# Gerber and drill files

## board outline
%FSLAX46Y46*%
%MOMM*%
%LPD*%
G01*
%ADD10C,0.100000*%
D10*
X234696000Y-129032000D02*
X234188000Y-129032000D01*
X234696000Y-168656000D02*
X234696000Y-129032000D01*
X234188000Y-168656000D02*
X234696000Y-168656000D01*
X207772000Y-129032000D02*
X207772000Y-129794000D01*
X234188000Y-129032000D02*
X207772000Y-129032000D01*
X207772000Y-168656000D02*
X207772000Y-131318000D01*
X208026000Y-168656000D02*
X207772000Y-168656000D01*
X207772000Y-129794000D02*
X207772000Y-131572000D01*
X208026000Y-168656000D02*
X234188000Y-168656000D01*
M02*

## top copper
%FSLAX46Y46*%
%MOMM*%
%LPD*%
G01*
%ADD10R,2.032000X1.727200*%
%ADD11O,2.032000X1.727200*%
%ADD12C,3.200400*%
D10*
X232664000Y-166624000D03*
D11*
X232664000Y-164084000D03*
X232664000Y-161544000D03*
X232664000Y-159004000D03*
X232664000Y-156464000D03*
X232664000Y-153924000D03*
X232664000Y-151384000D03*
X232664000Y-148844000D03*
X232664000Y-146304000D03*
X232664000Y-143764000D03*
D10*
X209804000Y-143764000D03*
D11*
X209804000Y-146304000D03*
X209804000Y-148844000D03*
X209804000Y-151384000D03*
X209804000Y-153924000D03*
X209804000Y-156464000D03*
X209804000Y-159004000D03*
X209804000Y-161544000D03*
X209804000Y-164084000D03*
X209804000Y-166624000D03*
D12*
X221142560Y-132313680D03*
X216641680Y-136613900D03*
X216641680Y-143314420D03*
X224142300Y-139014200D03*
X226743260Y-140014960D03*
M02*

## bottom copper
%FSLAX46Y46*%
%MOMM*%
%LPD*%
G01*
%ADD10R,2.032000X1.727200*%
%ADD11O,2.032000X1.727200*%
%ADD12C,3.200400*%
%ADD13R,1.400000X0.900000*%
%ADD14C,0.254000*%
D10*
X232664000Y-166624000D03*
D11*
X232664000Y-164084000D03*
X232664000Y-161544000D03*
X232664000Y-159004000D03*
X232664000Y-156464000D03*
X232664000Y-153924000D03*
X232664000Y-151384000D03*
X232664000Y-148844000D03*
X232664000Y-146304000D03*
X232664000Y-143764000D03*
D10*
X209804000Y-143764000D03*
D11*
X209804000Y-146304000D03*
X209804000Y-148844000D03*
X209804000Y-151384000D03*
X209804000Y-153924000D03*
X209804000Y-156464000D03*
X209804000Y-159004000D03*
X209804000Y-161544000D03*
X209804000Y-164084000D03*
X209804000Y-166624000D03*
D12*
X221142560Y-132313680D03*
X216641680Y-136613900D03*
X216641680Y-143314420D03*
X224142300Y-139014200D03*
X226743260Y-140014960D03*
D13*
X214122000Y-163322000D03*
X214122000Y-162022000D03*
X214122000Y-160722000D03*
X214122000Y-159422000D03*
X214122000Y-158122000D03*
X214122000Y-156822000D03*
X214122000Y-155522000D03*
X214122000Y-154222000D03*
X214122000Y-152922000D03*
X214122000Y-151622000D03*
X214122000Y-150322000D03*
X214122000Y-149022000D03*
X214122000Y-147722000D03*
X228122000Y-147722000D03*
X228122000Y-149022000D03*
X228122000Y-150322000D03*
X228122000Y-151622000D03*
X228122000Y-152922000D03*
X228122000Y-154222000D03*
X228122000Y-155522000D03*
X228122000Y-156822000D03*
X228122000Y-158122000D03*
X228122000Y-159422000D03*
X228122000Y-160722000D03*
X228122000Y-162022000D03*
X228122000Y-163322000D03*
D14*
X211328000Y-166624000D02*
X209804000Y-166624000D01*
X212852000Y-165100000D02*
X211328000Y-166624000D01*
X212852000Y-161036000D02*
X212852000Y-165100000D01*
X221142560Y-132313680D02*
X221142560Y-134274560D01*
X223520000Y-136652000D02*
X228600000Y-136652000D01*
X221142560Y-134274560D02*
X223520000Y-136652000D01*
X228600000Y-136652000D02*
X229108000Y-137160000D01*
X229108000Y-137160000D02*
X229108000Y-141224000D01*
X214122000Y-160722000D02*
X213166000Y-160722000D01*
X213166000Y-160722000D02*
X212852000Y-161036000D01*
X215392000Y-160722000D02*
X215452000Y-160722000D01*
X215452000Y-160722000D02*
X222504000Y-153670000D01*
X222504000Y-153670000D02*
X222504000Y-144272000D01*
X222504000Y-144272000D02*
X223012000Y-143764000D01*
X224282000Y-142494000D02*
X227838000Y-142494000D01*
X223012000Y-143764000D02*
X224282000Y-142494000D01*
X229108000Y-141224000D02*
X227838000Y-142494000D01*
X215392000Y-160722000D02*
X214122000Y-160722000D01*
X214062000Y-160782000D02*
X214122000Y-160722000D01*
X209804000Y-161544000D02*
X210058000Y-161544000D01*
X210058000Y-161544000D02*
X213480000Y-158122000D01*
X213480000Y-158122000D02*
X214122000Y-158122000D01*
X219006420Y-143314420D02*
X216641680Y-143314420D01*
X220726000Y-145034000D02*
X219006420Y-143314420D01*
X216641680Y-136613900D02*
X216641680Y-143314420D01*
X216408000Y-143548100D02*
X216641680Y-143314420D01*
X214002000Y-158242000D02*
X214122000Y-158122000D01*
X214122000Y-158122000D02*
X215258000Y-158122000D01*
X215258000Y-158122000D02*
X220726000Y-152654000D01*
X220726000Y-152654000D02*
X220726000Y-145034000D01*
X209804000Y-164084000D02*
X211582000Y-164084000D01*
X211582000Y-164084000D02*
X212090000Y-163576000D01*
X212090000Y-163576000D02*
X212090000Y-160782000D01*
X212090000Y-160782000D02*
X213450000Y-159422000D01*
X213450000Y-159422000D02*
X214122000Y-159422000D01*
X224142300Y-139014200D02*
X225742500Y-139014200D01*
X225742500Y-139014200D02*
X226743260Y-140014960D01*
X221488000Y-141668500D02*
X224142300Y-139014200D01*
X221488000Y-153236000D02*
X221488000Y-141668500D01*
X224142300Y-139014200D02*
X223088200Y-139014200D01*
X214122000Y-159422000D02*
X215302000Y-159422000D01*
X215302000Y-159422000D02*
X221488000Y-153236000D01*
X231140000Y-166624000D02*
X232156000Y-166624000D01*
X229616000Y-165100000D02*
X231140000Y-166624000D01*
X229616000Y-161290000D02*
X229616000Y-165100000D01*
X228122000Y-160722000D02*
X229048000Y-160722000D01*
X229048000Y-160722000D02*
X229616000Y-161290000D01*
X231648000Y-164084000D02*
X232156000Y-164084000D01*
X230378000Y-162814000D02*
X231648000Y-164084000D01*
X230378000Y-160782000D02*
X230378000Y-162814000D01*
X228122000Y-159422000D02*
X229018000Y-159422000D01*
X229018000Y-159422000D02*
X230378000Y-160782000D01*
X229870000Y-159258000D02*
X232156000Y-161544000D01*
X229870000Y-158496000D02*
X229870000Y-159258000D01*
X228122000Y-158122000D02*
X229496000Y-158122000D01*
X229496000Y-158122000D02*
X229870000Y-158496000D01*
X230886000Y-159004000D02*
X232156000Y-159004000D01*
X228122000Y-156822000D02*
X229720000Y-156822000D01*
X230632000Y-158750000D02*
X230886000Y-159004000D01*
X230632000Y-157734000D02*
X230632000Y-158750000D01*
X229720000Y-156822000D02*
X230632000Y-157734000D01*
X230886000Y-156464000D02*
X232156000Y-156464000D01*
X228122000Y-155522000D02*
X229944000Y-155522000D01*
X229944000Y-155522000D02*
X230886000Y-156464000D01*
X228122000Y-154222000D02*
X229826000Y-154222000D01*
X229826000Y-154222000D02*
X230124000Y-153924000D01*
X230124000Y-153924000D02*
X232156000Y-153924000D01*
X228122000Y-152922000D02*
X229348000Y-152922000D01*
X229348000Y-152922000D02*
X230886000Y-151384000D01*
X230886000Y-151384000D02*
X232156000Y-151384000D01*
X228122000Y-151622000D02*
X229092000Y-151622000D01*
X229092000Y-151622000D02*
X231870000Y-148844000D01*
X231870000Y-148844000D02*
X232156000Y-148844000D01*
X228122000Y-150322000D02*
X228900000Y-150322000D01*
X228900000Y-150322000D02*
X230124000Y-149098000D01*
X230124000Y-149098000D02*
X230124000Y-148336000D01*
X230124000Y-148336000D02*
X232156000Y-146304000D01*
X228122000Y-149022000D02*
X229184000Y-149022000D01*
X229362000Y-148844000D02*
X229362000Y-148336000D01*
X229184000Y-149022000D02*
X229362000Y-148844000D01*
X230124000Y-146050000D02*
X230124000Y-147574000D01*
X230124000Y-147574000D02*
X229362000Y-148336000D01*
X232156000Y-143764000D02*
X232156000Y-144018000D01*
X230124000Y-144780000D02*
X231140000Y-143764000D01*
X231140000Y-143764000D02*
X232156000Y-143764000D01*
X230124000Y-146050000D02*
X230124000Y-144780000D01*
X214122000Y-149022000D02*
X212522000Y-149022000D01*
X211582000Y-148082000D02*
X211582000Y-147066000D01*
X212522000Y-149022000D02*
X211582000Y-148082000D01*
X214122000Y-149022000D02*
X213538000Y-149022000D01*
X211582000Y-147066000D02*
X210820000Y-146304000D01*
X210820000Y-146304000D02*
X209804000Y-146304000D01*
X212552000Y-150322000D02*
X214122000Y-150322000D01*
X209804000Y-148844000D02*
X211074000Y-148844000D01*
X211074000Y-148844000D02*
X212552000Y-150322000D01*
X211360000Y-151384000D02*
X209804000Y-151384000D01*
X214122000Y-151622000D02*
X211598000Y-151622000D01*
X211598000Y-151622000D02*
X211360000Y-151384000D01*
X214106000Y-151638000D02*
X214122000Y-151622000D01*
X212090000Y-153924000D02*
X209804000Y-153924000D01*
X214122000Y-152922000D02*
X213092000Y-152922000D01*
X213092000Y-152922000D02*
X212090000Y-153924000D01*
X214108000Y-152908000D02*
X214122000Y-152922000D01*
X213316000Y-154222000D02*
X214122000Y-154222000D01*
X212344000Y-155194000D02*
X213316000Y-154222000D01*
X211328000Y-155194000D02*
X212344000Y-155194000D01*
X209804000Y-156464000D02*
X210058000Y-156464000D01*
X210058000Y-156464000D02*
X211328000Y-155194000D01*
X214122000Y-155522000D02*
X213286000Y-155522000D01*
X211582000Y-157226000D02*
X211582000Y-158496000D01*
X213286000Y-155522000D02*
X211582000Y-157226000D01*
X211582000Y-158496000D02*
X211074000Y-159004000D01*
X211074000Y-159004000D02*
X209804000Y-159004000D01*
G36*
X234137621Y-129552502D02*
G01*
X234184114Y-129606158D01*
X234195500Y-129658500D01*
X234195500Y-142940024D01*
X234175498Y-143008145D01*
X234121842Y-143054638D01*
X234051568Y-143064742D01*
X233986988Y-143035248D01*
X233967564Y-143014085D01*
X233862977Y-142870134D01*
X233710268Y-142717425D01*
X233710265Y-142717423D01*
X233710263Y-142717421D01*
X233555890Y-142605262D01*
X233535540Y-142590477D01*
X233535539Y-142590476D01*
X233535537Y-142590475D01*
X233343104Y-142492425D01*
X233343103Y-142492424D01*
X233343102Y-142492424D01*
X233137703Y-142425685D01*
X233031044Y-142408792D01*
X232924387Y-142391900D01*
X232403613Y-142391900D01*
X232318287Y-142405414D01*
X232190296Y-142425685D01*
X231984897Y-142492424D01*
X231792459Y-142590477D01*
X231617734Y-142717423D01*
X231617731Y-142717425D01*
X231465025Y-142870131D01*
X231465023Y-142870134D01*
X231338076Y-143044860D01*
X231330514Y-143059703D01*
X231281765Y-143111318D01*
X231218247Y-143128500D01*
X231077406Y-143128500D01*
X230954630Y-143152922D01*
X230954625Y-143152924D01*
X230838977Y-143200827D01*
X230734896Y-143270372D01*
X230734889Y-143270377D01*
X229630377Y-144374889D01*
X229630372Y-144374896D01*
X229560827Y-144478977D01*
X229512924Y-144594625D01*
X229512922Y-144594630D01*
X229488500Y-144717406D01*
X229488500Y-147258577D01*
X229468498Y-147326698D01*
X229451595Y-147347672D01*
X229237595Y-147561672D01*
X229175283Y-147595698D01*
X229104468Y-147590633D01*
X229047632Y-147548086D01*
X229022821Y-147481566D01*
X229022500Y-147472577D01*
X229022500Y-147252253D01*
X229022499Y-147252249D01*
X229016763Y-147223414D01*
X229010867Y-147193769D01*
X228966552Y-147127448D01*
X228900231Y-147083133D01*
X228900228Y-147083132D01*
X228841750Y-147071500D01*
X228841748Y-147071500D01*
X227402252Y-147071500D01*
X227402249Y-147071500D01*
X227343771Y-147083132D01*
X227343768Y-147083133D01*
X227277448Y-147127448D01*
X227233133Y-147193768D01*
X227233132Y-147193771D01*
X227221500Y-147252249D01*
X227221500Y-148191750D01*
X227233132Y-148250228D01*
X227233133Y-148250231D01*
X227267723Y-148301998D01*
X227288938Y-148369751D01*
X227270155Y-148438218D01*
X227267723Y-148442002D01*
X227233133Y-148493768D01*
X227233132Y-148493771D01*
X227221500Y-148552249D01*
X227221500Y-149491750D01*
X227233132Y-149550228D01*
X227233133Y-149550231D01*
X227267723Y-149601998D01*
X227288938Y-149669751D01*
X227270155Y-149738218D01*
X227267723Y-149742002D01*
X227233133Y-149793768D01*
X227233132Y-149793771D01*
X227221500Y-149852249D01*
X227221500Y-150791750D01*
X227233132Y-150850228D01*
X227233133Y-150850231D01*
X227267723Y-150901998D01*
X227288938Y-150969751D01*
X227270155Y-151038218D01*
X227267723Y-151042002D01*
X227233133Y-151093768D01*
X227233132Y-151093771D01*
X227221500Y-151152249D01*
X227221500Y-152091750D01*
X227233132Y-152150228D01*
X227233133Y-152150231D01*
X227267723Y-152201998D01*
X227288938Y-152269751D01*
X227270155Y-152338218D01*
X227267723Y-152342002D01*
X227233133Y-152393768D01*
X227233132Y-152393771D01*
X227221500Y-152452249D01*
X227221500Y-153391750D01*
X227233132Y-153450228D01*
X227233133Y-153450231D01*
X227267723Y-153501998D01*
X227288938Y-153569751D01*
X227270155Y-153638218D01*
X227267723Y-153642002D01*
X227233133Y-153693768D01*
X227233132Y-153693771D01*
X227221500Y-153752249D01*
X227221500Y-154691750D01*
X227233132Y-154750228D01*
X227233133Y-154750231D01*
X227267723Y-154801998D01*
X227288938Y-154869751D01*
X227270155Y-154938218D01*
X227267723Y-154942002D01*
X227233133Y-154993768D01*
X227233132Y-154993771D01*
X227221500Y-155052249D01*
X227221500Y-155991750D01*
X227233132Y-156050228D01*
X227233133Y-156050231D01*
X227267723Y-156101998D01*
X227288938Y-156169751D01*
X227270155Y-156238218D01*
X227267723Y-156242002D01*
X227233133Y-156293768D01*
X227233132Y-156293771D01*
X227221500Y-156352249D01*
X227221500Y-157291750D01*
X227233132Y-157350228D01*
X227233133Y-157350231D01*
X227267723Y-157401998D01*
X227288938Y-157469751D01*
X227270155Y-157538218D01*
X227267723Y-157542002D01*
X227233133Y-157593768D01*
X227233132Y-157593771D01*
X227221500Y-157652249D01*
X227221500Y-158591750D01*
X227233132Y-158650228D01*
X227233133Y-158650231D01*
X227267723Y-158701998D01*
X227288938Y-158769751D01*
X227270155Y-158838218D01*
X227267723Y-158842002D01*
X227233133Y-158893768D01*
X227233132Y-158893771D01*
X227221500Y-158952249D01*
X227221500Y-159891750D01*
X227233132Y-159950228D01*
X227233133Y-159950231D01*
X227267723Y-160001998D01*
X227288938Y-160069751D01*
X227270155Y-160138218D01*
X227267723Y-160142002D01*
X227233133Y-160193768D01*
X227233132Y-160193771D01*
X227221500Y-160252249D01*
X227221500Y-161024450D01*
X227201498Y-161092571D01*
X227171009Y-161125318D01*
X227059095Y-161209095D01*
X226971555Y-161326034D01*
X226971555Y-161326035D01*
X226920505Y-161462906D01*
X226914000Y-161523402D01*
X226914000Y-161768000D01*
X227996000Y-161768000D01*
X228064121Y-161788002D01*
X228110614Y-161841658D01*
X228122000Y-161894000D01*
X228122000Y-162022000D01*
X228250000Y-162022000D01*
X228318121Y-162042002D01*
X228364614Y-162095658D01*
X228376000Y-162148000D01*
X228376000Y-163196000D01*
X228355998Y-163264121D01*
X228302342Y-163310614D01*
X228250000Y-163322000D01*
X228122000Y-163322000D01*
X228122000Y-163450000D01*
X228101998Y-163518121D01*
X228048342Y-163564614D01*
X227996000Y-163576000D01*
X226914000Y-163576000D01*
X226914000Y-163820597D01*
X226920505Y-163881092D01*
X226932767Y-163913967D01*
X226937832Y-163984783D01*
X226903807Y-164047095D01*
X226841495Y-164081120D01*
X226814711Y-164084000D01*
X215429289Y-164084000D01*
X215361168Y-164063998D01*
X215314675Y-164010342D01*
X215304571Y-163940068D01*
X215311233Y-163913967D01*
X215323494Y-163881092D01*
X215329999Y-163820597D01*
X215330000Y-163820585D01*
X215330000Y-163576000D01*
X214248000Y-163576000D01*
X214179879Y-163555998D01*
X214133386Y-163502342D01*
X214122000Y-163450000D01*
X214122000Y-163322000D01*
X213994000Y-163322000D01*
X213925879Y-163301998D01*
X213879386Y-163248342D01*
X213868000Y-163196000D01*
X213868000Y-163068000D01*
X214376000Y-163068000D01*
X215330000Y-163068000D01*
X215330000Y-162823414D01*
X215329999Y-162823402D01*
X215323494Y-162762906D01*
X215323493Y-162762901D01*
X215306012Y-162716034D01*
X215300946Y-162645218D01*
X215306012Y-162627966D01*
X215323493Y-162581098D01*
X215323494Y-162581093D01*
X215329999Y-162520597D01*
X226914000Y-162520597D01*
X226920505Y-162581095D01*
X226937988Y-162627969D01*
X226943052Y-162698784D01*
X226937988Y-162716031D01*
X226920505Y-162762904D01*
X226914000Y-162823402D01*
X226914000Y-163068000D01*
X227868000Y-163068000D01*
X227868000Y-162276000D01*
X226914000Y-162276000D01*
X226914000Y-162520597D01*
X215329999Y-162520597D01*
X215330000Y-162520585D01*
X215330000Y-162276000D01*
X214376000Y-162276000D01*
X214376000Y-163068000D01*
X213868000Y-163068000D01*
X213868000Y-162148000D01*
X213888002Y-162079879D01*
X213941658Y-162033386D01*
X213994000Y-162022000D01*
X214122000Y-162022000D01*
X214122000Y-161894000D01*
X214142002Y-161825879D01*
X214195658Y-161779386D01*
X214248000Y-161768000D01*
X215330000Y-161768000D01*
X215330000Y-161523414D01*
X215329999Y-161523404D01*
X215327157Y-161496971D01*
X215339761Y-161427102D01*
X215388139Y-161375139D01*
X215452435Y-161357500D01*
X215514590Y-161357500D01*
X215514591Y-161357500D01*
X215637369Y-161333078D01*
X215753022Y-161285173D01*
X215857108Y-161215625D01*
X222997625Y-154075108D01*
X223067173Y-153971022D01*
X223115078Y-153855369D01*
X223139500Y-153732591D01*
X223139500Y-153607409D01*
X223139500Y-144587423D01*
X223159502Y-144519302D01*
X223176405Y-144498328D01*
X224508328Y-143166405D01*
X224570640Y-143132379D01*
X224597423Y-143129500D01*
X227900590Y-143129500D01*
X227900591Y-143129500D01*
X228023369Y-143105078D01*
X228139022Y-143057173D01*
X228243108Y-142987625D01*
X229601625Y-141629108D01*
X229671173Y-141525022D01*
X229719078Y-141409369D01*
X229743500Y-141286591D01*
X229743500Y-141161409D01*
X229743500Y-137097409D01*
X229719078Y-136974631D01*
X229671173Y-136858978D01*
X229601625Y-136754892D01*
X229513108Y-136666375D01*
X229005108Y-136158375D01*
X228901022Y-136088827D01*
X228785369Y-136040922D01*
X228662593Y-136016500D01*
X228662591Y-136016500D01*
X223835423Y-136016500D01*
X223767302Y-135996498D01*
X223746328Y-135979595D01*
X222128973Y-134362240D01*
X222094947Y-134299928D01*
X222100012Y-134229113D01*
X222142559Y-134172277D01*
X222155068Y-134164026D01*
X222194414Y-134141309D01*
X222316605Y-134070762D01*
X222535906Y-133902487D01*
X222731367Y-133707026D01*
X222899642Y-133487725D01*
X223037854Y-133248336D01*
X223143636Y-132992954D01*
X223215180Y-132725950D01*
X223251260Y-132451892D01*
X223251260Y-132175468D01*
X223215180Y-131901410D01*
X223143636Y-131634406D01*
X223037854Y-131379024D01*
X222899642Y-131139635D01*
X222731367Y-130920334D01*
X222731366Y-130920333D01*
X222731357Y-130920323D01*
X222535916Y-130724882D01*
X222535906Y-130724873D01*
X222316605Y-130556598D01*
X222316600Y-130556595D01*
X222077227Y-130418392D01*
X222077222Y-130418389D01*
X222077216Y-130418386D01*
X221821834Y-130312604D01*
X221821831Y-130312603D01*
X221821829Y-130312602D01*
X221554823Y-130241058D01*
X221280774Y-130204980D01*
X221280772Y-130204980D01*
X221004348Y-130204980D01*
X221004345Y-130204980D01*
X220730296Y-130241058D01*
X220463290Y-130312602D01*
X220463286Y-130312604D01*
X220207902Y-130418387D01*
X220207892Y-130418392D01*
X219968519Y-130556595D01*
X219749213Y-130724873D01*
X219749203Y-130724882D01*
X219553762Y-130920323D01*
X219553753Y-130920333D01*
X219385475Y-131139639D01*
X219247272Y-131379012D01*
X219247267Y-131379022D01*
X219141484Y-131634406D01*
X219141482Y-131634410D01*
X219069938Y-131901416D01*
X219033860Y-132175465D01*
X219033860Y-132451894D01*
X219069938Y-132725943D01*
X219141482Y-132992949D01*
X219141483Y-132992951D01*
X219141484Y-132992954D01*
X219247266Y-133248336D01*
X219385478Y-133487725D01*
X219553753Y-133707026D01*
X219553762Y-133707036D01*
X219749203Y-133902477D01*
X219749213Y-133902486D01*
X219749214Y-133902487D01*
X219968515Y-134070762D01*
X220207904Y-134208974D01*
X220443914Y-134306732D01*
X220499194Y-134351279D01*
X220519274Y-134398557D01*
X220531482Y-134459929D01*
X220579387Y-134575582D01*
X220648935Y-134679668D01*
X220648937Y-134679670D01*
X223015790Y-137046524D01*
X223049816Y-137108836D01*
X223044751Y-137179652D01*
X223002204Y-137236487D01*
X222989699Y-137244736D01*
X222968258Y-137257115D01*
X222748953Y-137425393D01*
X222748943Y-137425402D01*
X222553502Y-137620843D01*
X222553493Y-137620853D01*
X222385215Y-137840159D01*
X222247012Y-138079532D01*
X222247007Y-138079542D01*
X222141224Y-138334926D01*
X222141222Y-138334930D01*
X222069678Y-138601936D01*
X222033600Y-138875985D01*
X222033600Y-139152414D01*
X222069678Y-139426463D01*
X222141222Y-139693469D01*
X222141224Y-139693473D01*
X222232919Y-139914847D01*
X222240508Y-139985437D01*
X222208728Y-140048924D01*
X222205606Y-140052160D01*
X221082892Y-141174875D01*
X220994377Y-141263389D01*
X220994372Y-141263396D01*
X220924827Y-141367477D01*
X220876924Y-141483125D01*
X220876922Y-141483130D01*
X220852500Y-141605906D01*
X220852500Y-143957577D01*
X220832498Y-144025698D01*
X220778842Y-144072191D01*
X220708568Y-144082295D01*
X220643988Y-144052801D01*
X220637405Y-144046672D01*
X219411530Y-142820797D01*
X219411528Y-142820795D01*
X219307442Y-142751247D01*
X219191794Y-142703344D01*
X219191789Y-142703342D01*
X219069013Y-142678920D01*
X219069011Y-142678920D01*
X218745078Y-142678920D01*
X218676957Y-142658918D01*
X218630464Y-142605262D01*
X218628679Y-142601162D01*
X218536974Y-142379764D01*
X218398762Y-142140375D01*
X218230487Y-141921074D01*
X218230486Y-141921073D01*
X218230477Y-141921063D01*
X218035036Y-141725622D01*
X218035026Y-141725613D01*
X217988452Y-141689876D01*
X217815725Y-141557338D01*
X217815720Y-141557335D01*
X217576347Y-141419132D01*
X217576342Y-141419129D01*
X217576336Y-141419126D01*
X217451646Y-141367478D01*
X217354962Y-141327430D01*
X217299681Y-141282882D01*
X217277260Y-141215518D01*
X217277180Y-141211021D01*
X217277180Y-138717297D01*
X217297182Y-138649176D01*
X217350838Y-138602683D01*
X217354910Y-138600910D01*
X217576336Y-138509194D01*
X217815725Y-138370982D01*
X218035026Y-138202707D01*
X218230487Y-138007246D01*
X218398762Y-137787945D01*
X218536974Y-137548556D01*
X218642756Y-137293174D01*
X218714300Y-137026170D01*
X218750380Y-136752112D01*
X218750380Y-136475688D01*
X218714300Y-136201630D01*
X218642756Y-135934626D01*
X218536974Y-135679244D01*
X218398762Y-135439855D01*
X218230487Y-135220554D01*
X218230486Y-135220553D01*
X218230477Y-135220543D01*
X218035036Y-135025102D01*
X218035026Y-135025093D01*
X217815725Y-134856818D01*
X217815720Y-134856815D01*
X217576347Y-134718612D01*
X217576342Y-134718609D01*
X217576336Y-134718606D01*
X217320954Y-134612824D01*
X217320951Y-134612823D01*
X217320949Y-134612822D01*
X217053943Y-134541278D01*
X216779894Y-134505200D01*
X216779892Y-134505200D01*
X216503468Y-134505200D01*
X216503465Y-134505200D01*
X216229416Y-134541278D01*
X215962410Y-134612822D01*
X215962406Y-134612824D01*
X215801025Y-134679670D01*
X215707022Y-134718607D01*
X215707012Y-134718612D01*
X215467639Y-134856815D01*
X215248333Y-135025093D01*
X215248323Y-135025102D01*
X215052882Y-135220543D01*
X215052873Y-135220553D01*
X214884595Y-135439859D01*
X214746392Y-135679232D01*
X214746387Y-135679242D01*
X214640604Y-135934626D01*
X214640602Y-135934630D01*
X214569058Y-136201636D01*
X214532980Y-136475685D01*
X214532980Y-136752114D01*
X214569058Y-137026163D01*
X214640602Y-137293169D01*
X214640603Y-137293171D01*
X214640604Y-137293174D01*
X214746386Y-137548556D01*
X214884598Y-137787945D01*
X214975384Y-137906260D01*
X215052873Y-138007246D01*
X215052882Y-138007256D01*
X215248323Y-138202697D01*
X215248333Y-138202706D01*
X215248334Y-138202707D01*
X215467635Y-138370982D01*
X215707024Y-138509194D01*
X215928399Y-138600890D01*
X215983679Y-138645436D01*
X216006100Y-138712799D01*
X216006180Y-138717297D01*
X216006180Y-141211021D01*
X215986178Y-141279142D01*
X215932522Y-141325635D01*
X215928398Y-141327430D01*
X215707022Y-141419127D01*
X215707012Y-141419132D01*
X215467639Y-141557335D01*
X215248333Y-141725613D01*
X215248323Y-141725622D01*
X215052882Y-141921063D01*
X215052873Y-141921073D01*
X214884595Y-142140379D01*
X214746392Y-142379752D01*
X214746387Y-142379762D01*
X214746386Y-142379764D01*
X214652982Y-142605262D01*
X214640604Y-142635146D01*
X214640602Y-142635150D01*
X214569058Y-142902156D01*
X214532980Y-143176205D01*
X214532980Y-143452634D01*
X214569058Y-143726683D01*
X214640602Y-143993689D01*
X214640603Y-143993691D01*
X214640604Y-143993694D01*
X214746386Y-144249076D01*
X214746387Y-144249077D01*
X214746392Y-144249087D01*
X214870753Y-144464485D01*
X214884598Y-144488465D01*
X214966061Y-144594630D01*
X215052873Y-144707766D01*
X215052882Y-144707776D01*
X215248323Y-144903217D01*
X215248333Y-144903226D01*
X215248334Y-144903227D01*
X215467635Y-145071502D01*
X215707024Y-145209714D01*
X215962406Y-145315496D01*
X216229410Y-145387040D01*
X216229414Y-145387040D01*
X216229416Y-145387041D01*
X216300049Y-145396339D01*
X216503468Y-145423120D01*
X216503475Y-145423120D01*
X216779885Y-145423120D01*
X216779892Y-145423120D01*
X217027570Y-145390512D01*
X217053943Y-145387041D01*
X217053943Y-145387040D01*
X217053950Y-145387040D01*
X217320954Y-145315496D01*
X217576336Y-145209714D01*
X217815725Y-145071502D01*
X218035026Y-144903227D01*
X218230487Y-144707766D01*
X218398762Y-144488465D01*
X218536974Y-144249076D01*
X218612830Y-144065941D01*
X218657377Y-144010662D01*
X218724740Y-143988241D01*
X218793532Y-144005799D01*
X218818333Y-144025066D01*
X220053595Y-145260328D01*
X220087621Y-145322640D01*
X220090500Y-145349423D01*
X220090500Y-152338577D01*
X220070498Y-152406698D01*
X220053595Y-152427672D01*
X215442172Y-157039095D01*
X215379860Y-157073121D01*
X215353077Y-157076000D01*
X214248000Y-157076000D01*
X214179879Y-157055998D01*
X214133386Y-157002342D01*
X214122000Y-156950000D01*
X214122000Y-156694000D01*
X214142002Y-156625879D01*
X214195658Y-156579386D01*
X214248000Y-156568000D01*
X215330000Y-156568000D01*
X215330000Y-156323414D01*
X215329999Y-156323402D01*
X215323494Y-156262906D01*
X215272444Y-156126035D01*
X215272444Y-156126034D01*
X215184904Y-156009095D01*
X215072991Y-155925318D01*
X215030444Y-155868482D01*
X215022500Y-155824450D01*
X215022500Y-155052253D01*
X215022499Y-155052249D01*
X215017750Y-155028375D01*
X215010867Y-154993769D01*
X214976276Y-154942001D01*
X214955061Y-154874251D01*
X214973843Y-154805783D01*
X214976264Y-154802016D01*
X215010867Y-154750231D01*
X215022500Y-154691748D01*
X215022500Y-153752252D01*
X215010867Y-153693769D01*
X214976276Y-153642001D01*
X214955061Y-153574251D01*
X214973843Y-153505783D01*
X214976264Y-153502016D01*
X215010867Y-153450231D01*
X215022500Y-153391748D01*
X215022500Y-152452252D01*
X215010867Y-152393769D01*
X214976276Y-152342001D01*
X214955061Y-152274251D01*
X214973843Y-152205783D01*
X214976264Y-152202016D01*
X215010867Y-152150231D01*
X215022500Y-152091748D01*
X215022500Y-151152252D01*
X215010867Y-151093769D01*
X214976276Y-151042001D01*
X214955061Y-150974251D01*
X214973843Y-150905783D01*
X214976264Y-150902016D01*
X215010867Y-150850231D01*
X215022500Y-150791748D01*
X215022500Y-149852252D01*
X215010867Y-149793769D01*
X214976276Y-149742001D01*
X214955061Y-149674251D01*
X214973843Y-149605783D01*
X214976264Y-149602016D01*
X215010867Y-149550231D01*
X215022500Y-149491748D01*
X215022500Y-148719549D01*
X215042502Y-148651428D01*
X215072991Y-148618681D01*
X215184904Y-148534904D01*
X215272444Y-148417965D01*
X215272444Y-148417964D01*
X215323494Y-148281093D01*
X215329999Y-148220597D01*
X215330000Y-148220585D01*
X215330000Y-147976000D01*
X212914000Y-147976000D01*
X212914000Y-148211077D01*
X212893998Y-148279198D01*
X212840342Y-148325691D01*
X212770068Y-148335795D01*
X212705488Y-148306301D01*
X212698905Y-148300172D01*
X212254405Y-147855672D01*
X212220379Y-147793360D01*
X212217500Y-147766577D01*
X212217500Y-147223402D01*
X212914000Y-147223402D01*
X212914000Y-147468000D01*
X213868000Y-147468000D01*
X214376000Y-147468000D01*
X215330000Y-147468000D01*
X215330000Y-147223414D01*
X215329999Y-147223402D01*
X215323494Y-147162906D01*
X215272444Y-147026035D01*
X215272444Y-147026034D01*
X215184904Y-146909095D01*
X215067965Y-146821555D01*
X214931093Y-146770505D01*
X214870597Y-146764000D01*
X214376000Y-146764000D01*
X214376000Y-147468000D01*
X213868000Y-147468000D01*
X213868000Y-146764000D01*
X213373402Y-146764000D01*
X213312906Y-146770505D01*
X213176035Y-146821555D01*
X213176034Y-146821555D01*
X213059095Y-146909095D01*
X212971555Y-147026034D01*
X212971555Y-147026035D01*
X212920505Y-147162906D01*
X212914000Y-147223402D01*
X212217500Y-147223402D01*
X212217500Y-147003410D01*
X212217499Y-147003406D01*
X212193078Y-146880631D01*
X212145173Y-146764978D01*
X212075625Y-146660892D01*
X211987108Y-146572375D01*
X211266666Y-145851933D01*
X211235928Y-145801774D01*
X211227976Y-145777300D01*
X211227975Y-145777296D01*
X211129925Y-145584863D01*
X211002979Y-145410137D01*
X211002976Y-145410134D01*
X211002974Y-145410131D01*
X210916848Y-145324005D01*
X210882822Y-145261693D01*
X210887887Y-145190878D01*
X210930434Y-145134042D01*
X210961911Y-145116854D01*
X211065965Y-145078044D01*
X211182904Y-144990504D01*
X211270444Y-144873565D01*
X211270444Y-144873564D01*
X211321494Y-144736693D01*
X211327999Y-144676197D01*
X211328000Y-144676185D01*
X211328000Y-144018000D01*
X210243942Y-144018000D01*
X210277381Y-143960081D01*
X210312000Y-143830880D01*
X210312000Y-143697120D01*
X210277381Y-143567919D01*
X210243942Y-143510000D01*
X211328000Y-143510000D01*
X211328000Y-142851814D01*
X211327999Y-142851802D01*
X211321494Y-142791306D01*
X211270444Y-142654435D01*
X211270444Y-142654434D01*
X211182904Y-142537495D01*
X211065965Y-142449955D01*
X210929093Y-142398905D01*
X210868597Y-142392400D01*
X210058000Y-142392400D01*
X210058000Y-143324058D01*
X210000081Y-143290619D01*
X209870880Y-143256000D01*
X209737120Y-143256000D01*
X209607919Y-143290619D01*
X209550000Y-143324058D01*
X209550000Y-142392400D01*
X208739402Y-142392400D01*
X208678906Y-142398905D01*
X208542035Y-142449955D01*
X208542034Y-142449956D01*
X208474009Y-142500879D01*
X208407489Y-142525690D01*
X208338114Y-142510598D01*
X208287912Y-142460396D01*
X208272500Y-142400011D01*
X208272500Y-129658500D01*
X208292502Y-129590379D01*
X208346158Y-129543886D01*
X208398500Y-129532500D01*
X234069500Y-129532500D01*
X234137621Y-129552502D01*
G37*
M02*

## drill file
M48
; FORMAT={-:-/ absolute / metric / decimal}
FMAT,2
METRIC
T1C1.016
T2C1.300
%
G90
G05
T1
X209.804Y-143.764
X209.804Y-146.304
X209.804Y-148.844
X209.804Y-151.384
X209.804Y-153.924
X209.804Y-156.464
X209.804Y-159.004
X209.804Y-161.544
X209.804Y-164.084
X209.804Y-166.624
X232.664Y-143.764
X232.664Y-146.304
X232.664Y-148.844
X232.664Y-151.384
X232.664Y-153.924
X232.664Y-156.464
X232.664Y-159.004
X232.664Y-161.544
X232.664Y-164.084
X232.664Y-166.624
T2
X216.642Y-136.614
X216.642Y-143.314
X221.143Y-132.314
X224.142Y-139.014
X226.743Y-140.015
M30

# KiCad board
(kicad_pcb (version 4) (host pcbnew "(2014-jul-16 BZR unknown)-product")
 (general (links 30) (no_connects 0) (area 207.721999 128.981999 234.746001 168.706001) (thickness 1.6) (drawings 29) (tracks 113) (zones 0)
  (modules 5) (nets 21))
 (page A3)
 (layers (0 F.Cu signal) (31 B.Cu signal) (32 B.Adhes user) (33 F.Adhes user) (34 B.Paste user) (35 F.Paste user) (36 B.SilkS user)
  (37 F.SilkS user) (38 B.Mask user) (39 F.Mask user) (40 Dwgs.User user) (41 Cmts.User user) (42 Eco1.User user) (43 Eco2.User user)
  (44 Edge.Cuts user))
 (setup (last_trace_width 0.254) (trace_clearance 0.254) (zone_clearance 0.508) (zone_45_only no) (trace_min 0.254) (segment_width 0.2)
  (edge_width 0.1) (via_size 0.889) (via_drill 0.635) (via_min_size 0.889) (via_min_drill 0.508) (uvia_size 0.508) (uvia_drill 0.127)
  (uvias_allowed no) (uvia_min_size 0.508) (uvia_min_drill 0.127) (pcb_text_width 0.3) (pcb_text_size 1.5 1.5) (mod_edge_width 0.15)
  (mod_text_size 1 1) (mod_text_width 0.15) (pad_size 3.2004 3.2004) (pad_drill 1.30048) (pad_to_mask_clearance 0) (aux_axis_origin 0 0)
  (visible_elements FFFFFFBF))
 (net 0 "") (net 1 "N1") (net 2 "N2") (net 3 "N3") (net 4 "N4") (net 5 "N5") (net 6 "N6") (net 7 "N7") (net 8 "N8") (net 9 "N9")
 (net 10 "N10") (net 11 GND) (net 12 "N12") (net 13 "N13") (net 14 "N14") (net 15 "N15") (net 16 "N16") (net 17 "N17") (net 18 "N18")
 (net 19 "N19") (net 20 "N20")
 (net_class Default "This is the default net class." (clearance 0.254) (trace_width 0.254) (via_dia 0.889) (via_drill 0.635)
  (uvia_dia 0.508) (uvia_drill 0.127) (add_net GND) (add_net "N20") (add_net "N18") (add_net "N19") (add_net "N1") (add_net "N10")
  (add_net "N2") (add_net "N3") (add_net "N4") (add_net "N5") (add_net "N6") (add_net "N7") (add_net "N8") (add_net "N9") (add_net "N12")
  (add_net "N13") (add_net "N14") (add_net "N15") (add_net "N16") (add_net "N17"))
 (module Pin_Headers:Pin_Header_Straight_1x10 (layer B.Cu) (at 232.664 155.194 90)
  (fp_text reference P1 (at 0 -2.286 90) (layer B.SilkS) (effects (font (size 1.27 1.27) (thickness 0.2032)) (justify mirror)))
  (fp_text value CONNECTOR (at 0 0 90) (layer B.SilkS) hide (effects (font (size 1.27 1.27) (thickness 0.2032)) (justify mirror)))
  (pad 1 thru_hole rect (at -11.43 0 90) (size 1.7272 2.032) (drill 1.016) (layers *.Cu *.Mask B.SilkS) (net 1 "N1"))
  (pad 2 thru_hole oval (at -8.89 0 90) (size 1.7272 2.032) (drill 1.016) (layers *.Cu *.Mask B.SilkS) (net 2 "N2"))
  (pad 3 thru_hole oval (at -6.35 0 90) (size 1.7272 2.032) (drill 1.016) (layers *.Cu *.Mask B.SilkS) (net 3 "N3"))
  (pad 4 thru_hole oval (at -3.81 0 90) (size 1.7272 2.032) (drill 1.016) (layers *.Cu *.Mask B.SilkS) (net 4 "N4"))
  (pad 5 thru_hole oval (at -1.27 0 90) (size 1.7272 2.032) (drill 1.016) (layers *.Cu *.Mask B.SilkS) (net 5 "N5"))
  (pad 6 thru_hole oval (at 1.27 0 90) (size 1.7272 2.032) (drill 1.016) (layers *.Cu *.Mask B.SilkS) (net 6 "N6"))
  (pad 7 thru_hole oval (at 3.81 0 90) (size 1.7272 2.032) (drill 1.016) (layers *.Cu *.Mask B.SilkS) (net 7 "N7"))
  (pad 8 thru_hole oval (at 6.35 0 90) (size 1.7272 2.032) (drill 1.016) (layers *.Cu *.Mask B.SilkS) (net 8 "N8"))
  (pad 9 thru_hole oval (at 8.89 0 90) (size 1.7272 2.032) (drill 1.016) (layers *.Cu *.Mask B.SilkS) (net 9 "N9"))
  (pad 10 thru_hole oval (at 11.43 0 90) (size 1.7272 2.032) (drill 1.016) (layers *.Cu *.Mask B.SilkS) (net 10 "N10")))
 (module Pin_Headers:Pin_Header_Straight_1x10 (layer B.Cu) (at 209.804 155.194 270)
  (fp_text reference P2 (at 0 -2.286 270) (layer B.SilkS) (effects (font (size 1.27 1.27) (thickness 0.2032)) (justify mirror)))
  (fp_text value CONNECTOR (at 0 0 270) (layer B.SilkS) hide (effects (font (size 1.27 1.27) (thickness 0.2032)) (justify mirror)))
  (pad 1 thru_hole rect (at -11.43 0 270) (size 1.7272 2.032) (drill 1.016) (layers *.Cu *.Mask B.SilkS) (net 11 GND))
  (pad 2 thru_hole oval (at -8.89 0 270) (size 1.7272 2.032) (drill 1.016) (layers *.Cu *.Mask B.SilkS) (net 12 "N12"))
  (pad 3 thru_hole oval (at -6.35 0 270) (size 1.7272 2.032) (drill 1.016) (layers *.Cu *.Mask B.SilkS) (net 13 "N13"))
  (pad 4 thru_hole oval (at -3.81 0 270) (size 1.7272 2.032) (drill 1.016) (layers *.Cu *.Mask B.SilkS) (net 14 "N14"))
  (pad 5 thru_hole oval (at -1.27 0 270) (size 1.7272 2.032) (drill 1.016) (layers *.Cu *.Mask B.SilkS) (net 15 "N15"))
  (pad 6 thru_hole oval (at 1.27 0 270) (size 1.7272 2.032) (drill 1.016) (layers *.Cu *.Mask B.SilkS) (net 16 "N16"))
  (pad 7 thru_hole oval (at 3.81 0 270) (size 1.7272 2.032) (drill 1.016) (layers *.Cu *.Mask B.SilkS) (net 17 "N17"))
  (pad 8 thru_hole oval (at 6.35 0 270) (size 1.7272 2.032) (drill 1.016) (layers *.Cu *.Mask B.SilkS) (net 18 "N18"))
  (pad 9 thru_hole oval (at 8.89 0 270) (size 1.7272 2.032) (drill 1.016) (layers *.Cu *.Mask B.SilkS) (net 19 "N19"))
  (pad 10 thru_hole oval (at 11.43 0 270) (size 1.7272 2.032) (drill 1.016) (layers *.Cu *.Mask B.SilkS) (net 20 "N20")))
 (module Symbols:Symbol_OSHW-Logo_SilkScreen (layer F.Cu) (at 211.582 132.842)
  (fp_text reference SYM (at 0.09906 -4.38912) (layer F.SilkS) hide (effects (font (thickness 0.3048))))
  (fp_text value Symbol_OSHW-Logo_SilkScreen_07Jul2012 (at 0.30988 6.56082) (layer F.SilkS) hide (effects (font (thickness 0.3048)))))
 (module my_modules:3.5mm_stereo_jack (layer F.Cu) (at 221.742 137.414)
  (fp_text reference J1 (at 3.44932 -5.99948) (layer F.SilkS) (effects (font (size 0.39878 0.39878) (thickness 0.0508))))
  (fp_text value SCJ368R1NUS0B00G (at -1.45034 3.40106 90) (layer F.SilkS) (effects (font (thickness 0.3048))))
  (pad 1 thru_hole circle (at -0.59944 -5.10032) (size 3.2004 3.2004) (drill 1.30048) (layers *.Cu *.Mask F.SilkS) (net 20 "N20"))
  (pad 2 thru_hole circle (at -5.10032 -0.8001) (size 3.2004 3.2004) (drill 1.30048) (layers *.Cu *.Mask F.SilkS) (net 18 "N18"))
  (pad 3 thru_hole circle (at -5.10032 5.90042) (size 3.2004 3.2004) (drill 1.30048) (layers *.Cu *.Mask F.SilkS) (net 18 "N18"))
  (pad 5 thru_hole circle (at 2.4003 1.6002) (size 3.2004 3.2004) (drill 1.30048) (layers *.Cu *.Mask F.SilkS) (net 19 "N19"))
  (pad 4 thru_hole circle (at 5.00126 2.60096) (size 3.2004 3.2004) (drill 1.30048) (layers *.Cu *.Mask F.SilkS) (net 19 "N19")))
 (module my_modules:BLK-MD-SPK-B (layer B.Cu) (at 212.852 169.672) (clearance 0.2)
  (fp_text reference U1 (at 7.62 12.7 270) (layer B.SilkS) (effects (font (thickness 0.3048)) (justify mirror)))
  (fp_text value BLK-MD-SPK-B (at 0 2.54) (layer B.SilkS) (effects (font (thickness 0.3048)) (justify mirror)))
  (pad 1 smd rect (at 1.27 -6.35 180) (size 1.4 0.9) (layers B.Cu B.Paste B.Mask) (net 11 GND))
  (pad 2 smd rect (at 1.27 -7.65 180) (size 1.4 0.9) (layers B.Cu B.Paste B.Mask) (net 11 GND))
  (pad 3 smd rect (at 1.27 -8.95 180) (size 1.4 0.9) (layers B.Cu B.Paste B.Mask) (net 20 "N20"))
  (pad 4 smd rect (at 1.27 -10.25 180) (size 1.4 0.9) (layers B.Cu B.Paste B.Mask) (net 19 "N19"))
  (pad 5 smd rect (at 1.27 -11.55 180) (size 1.4 0.9) (layers B.Cu B.Paste B.Mask) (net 18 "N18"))
  (pad 6 smd rect (at 1.27 -12.85 180) (size 1.4 0.9) (layers B.Cu B.Paste B.Mask) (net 11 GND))
  (pad 7 smd rect (at 1.27 -14.15 180) (size 1.4 0.9) (layers B.Cu B.Paste B.Mask) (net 17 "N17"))
  (pad 8 smd rect (at 1.27 -15.45 180) (size 1.4 0.9) (layers B.Cu B.Paste B.Mask) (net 16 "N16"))
  (pad 9 smd rect (at 1.27 -16.75 180) (size 1.4 0.9) (layers B.Cu B.Paste B.Mask) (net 15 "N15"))
  (pad 10 smd rect (at 1.27 -18.05 180) (size 1.4 0.9) (layers B.Cu B.Paste B.Mask) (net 14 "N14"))
  (pad 11 smd rect (at 1.27 -19.35 180) (size 1.4 0.9) (layers B.Cu B.Paste B.Mask) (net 13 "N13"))
  (pad 12 smd rect (at 1.27 -20.65 180) (size 1.4 0.9) (layers B.Cu B.Paste B.Mask) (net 12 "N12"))
  (pad 13 smd rect (at 1.27 -21.95 180) (size 1.4 0.9) (layers B.Cu B.Paste B.Mask) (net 11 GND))
  (pad 14 smd rect (at 15.27 -21.95 180) (size 1.4 0.9) (layers B.Cu B.Paste B.Mask))
  (pad 15 smd rect (at 15.27 -20.65 180) (size 1.4 0.9) (layers B.Cu B.Paste B.Mask) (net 10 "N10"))
  (pad 16 smd rect (at 15.27 -19.35 180) (size 1.4 0.9) (layers B.Cu B.Paste B.Mask) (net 9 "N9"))
  (pad 17 smd rect (at 15.27 -18.05 180) (size 1.4 0.9) (layers B.Cu B.Paste B.Mask) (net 8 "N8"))
  (pad 18 smd rect (at 15.27 -16.75 180) (size 1.4 0.9) (layers B.Cu B.Paste B.Mask) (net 7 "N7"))
  (pad 19 smd rect (at 15.27 -15.45 180) (size 1.4 0.9) (layers B.Cu B.Paste B.Mask) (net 6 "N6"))
  (pad 20 smd rect (at 15.27 -14.15 180) (size 1.4 0.9) (layers B.Cu B.Paste B.Mask) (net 5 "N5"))
  (pad 21 smd rect (at 15.27 -12.85 180) (size 1.4 0.9) (layers B.Cu B.Paste B.Mask) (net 4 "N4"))
  (pad 22 smd rect (at 15.27 -11.55 180) (size 1.4 0.9) (layers B.Cu B.Paste B.Mask) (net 3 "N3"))
  (pad 23 smd rect (at 15.27 -10.25 180) (size 1.4 0.9) (layers B.Cu B.Paste B.Mask) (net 2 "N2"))
  (pad 24 smd rect (at 15.27 -8.95 180) (size 1.4 0.9) (layers B.Cu B.Paste B.Mask) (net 1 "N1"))
  (pad 25 smd rect (at 15.27 -7.65 180) (size 1.4 0.9) (layers B.Cu B.Paste B.Mask) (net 11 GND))
  (pad 26 smd rect (at 15.27 -6.35 180) (size 1.4 0.9) (layers B.Cu B.Paste B.Mask) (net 11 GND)))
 (gr_line (start 234.696 129.032) (end 234.188 129.032) (angle 90) (layer Edge.Cuts) (width 0.1))
 (gr_line (start 234.696 168.656) (end 234.696 129.032) (angle 90) (layer Edge.Cuts) (width 0.1))
 (gr_line (start 234.188 168.656) (end 234.696 168.656) (angle 90) (layer Edge.Cuts) (width 0.1))
 (gr_line (start 207.772 129.032) (end 207.772 129.794) (angle 90) (layer Edge.Cuts) (width 0.1))
 (gr_line (start 234.188 129.032) (end 207.772 129.032) (angle 90) (layer Edge.Cuts) (width 0.1))
 (gr_line (start 207.772 168.656) (end 207.772 131.318) (angle 90) (layer Edge.Cuts) (width 0.1))
 (gr_line (start 208.026 168.656) (end 207.772 168.656) (angle 90) (layer Edge.Cuts) (width 0.1))
 (gr_line (start 207.772 129.794) (end 207.772 131.572) (angle 90) (layer Edge.Cuts) (width 0.1))
 (gr_line (start 208.026 168.656) (end 234.188 168.656) (angle 90) (layer Edge.Cuts) (width 0.1))
 (segment (start 211.328 166.624) (end 209.804 166.624) (width 0.254) (layer B.Cu) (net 20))
 (segment (start 212.852 165.1) (end 211.328 166.624) (width 0.254) (layer B.Cu) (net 20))
 (segment (start 212.852 161.036) (end 212.852 165.1) (width 0.254) (layer B.Cu) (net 20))
 (segment (start 221.14256 132.31368) (end 221.14256 134.27456) (width 0.254) (layer B.Cu) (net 20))
 (segment (start 223.52 136.652) (end 228.6 136.652) (width 0.254) (layer B.Cu) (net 20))
 (segment (start 221.14256 134.27456) (end 223.52 136.652) (width 0.254) (layer B.Cu) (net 20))
 (segment (start 228.6 136.652) (end 229.108 137.16) (width 0.254) (layer B.Cu) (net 20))
 (segment (start 229.108 137.16) (end 229.108 141.224) (width 0.254) (layer B.Cu) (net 20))
 (segment (start 214.122 160.722) (end 213.166 160.722) (width 0.254) (layer B.Cu) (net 20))
 (segment (start 213.166 160.722) (end 212.852 161.036) (width 0.254) (layer B.Cu) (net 20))
 (segment (start 215.392 160.722) (end 215.452 160.722) (width 0.254) (layer B.Cu) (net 20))
 (segment (start 215.452 160.722) (end 222.504 153.67) (width 0.254) (layer B.Cu) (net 20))
 (segment (start 222.504 153.67) (end 222.504 144.272) (width 0.254) (layer B.Cu) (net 20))
 (segment (start 222.504 144.272) (end 223.012 143.764) (width 0.254) (layer B.Cu) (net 20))
 (segment (start 224.282 142.494) (end 227.838 142.494) (width 0.254) (layer B.Cu) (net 20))
 (segment (start 223.012 143.764) (end 224.282 142.494) (width 0.254) (layer B.Cu) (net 20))
 (segment (start 229.108 141.224) (end 227.838 142.494) (width 0.254) (layer B.Cu) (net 20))
 (segment (start 215.392 160.722) (end 214.122 160.722) (width 0.254) (layer B.Cu) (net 20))
 (segment (start 214.062 160.782) (end 214.122 160.722) (width 0.254) (layer B.Cu) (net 20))
 (segment (start 209.804 161.544) (end 210.058 161.544) (width 0.254) (layer B.Cu) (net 18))
 (segment (start 210.058 161.544) (end 213.48 158.122) (width 0.254) (layer B.Cu) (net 18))
 (segment (start 213.48 158.122) (end 214.122 158.122) (width 0.254) (layer B.Cu) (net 18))
 (segment (start 219.00642 143.31442) (end 216.64168 143.31442) (width 0.254) (layer B.Cu) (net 18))
 (segment (start 220.726 145.034) (end 219.00642 143.31442) (width 0.254) (layer B.Cu) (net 18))
 (segment (start 216.64168 136.6139) (end 216.64168 143.31442) (width 0.254) (layer B.Cu) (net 18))
 (segment (start 216.408 143.5481) (end 216.64168 143.31442) (width 0.254) (layer B.Cu) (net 18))
 (segment (start 214.002 158.242) (end 214.122 158.122) (width 0.254) (layer B.Cu) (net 18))
 (segment (start 214.122 158.122) (end 215.258 158.122) (width 0.254) (layer B.Cu) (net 18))
 (segment (start 215.258 158.122) (end 220.726 152.654) (width 0.254) (layer B.Cu) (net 18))
 (segment (start 220.726 152.654) (end 220.726 145.034) (width 0.254) (layer B.Cu) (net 18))
 (segment (start 209.804 164.084) (end 211.582 164.084) (width 0.254) (layer B.Cu) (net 19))
 (segment (start 211.582 164.084) (end 212.09 163.576) (width 0.254) (layer B.Cu) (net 19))
 (segment (start 212.09 163.576) (end 212.09 160.782) (width 0.254) (layer B.Cu) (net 19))
 (segment (start 212.09 160.782) (end 213.45 159.422) (width 0.254) (layer B.Cu) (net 19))
 (segment (start 213.45 159.422) (end 214.122 159.422) (width 0.254) (layer B.Cu) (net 19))
 (segment (start 224.1423 139.0142) (end 225.7425 139.0142) (width 0.254) (layer B.Cu) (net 19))
 (segment (start 225.7425 139.0142) (end 226.74326 140.01496) (width 0.254) (layer B.Cu) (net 19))
 (segment (start 221.488 141.6685) (end 224.1423 139.0142) (width 0.254) (layer B.Cu) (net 19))
 (segment (start 221.488 153.236) (end 221.488 141.6685) (width 0.254) (layer B.Cu) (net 19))
 (segment (start 224.1423 139.0142) (end 223.0882 139.0142) (width 0.254) (layer B.Cu) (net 19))
 (segment (start 214.122 159.422) (end 215.302 159.422) (width 0.254) (layer B.Cu) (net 19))
 (segment (start 215.302 159.422) (end 221.488 153.236) (width 0.254) (layer B.Cu) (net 19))
 (segment (start 231.14 166.624) (end 232.156 166.624) (width 0.254) (layer B.Cu) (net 1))
 (segment (start 229.616 165.1) (end 231.14 166.624) (width 0.254) (layer B.Cu) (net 1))
 (segment (start 229.616 161.29) (end 229.616 165.1) (width 0.254) (layer B.Cu) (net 1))
 (segment (start 228.122 160.722) (end 229.048 160.722) (width 0.254) (layer B.Cu) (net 1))
 (segment (start 229.048 160.722) (end 229.616 161.29) (width 0.254) (layer B.Cu) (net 1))
 (segment (start 231.648 164.084) (end 232.156 164.084) (width 0.254) (layer B.Cu) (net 2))
 (segment (start 230.378 162.814) (end 231.648 164.084) (width 0.254) (layer B.Cu) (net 2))
 (segment (start 230.378 160.782) (end 230.378 162.814) (width 0.254) (layer B.Cu) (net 2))
 (segment (start 228.122 159.422) (end 229.018 159.422) (width 0.254) (layer B.Cu) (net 2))
 (segment (start 229.018 159.422) (end 230.378 160.782) (width 0.254) (layer B.Cu) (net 2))
 (segment (start 229.87 159.258) (end 232.156 161.544) (width 0.254) (layer B.Cu) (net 3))
 (segment (start 229.87 158.496) (end 229.87 159.258) (width 0.254) (layer B.Cu) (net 3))
 (segment (start 228.122 158.122) (end 229.496 158.122) (width 0.254) (layer B.Cu) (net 3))
 (segment (start 229.496 158.122) (end 229.87 158.496) (width 0.254) (layer B.Cu) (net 3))
 (segment (start 230.886 159.004) (end 232.156 159.004) (width 0.254) (layer B.Cu) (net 4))
 (segment (start 228.122 156.822) (end 229.72 156.822) (width 0.254) (layer B.Cu) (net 4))
 (segment (start 230.632 158.75) (end 230.886 159.004) (width 0.254) (layer B.Cu) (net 4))
 (segment (start 230.632 157.734) (end 230.632 158.75) (width 0.254) (layer B.Cu) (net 4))
 (segment (start 229.72 156.822) (end 230.632 157.734) (width 0.254) (layer B.Cu) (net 4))
 (segment (start 230.886 156.464) (end 232.156 156.464) (width 0.254) (layer B.Cu) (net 5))
 (segment (start 228.122 155.522) (end 229.944 155.522) (width 0.254) (layer B.Cu) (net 5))
 (segment (start 229.944 155.522) (end 230.886 156.464) (width 0.254) (layer B.Cu) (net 5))
 (segment (start 228.122 154.222) (end 229.826 154.222) (width 0.254) (layer B.Cu) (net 6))
 (segment (start 229.826 154.222) (end 230.124 153.924) (width 0.254) (layer B.Cu) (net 6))
 (segment (start 230.124 153.924) (end 232.156 153.924) (width 0.254) (layer B.Cu) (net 6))
 (segment (start 228.122 152.922) (end 229.348 152.922) (width 0.254) (layer B.Cu) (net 7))
 (segment (start 229.348 152.922) (end 230.886 151.384) (width 0.254) (layer B.Cu) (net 7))
 (segment (start 230.886 151.384) (end 232.156 151.384) (width 0.254) (layer B.Cu) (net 7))
 (segment (start 228.122 151.622) (end 229.092 151.622) (width 0.254) (layer B.Cu) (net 8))
 (segment (start 229.092 151.622) (end 231.87 148.844) (width 0.254) (layer B.Cu) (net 8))
 (segment (start 231.87 148.844) (end 232.156 148.844) (width 0.254) (layer B.Cu) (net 8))
 (segment (start 228.122 150.322) (end 228.9 150.322) (width 0.254) (layer B.Cu) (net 9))
 (segment (start 228.9 150.322) (end 230.124 149.098) (width 0.254) (layer B.Cu) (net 9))
 (segment (start 230.124 149.098) (end 230.124 148.336) (width 0.254) (layer B.Cu) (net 9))
 (segment (start 230.124 148.336) (end 232.156 146.304) (width 0.254) (layer B.Cu) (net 9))
 (segment (start 228.122 149.022) (end 229.184 149.022) (width 0.254) (layer B.Cu) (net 10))
 (segment (start 229.362 148.844) (end 229.362 148.336) (width 0.254) (layer B.Cu) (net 10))
 (segment (start 229.184 149.022) (end 229.362 148.844) (width 0.254) (layer B.Cu) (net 10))
 (segment (start 230.124 146.05) (end 230.124 147.574) (width 0.254) (layer B.Cu) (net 10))
 (segment (start 230.124 147.574) (end 229.362 148.336) (width 0.254) (layer B.Cu) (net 10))
 (segment (start 232.156 143.764) (end 232.156 144.018) (width 0.254) (layer B.Cu) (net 10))
 (segment (start 230.124 144.78) (end 231.14 143.764) (width 0.254) (layer B.Cu) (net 10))
 (segment (start 231.14 143.764) (end 232.156 143.764) (width 0.254) (layer B.Cu) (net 10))
 (segment (start 230.124 146.05) (end 230.124 144.78) (width 0.254) (layer B.Cu) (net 10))
 (segment (start 214.122 149.022) (end 212.522 149.022) (width 0.254) (layer B.Cu) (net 12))
 (segment (start 211.582 148.082) (end 211.582 147.066) (width 0.254) (layer B.Cu) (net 12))
 (segment (start 212.522 149.022) (end 211.582 148.082) (width 0.254) (layer B.Cu) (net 12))
 (segment (start 214.122 149.022) (end 213.538 149.022) (width 0.254) (layer B.Cu) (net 12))
 (segment (start 211.582 147.066) (end 210.82 146.304) (width 0.254) (layer B.Cu) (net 12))
 (segment (start 210.82 146.304) (end 209.804 146.304) (width 0.254) (layer B.Cu) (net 12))
 (segment (start 212.552 150.322) (end 214.122 150.322) (width 0.254) (layer B.Cu) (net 13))
 (segment (start 209.804 148.844) (end 211.074 148.844) (width 0.254) (layer B.Cu) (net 13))
 (segment (start 211.074 148.844) (end 212.552 150.322) (width 0.254) (layer B.Cu) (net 13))
 (segment (start 211.36 151.384) (end 209.804 151.384) (width 0.254) (layer B.Cu) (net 14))
 (segment (start 214.122 151.622) (end 211.598 151.622) (width 0.254) (layer B.Cu) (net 14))
 (segment (start 211.598 151.622) (end 211.36 151.384) (width 0.254) (layer B.Cu) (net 14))
 (segment (start 214.106 151.638) (end 214.122 151.622) (width 0.254) (layer B.Cu) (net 14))
 (segment (start 212.09 153.924) (end 209.804 153.924) (width 0.254) (layer B.Cu) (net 15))
 (segment (start 214.122 152.922) (end 213.092 152.922) (width 0.254) (layer B.Cu) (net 15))
 (segment (start 213.092 152.922) (end 212.09 153.924) (width 0.254) (layer B.Cu) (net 15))
 (segment (start 214.108 152.908) (end 214.122 152.922) (width 0.254) (layer B.Cu) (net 15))
 (segment (start 213.316 154.222) (end 214.122 154.222) (width 0.254) (layer B.Cu) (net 16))
 (segment (start 212.344 155.194) (end 213.316 154.222) (width 0.254) (layer B.Cu) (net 16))
 (segment (start 211.328 155.194) (end 212.344 155.194) (width 0.254) (layer B.Cu) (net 16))
 (segment (start 209.804 156.464) (end 210.058 156.464) (width 0.254) (layer B.Cu) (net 16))
 (segment (start 210.058 156.464) (end 211.328 155.194) (width 0.254) (layer B.Cu) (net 16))
 (segment (start 214.122 155.522) (end 213.286 155.522) (width 0.254) (layer B.Cu) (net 17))
 (segment (start 211.582 157.226) (end 211.582 158.496) (width 0.254) (layer B.Cu) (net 17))
 (segment (start 213.286 155.522) (end 211.582 157.226) (width 0.254) (layer B.Cu) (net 17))
 (segment (start 211.582 158.496) (end 211.074 159.004) (width 0.254) (layer B.Cu) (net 17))
 (segment (start 211.074 159.004) (end 209.804 159.004) (width 0.254) (layer B.Cu) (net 17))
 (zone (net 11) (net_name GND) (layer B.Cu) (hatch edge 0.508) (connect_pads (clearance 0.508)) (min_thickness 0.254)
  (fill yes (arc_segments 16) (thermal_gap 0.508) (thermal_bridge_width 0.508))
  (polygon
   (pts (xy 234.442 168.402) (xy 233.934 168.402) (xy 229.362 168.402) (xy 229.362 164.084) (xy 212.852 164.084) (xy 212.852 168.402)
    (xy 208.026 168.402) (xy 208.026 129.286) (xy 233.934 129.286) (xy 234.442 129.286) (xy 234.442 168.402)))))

